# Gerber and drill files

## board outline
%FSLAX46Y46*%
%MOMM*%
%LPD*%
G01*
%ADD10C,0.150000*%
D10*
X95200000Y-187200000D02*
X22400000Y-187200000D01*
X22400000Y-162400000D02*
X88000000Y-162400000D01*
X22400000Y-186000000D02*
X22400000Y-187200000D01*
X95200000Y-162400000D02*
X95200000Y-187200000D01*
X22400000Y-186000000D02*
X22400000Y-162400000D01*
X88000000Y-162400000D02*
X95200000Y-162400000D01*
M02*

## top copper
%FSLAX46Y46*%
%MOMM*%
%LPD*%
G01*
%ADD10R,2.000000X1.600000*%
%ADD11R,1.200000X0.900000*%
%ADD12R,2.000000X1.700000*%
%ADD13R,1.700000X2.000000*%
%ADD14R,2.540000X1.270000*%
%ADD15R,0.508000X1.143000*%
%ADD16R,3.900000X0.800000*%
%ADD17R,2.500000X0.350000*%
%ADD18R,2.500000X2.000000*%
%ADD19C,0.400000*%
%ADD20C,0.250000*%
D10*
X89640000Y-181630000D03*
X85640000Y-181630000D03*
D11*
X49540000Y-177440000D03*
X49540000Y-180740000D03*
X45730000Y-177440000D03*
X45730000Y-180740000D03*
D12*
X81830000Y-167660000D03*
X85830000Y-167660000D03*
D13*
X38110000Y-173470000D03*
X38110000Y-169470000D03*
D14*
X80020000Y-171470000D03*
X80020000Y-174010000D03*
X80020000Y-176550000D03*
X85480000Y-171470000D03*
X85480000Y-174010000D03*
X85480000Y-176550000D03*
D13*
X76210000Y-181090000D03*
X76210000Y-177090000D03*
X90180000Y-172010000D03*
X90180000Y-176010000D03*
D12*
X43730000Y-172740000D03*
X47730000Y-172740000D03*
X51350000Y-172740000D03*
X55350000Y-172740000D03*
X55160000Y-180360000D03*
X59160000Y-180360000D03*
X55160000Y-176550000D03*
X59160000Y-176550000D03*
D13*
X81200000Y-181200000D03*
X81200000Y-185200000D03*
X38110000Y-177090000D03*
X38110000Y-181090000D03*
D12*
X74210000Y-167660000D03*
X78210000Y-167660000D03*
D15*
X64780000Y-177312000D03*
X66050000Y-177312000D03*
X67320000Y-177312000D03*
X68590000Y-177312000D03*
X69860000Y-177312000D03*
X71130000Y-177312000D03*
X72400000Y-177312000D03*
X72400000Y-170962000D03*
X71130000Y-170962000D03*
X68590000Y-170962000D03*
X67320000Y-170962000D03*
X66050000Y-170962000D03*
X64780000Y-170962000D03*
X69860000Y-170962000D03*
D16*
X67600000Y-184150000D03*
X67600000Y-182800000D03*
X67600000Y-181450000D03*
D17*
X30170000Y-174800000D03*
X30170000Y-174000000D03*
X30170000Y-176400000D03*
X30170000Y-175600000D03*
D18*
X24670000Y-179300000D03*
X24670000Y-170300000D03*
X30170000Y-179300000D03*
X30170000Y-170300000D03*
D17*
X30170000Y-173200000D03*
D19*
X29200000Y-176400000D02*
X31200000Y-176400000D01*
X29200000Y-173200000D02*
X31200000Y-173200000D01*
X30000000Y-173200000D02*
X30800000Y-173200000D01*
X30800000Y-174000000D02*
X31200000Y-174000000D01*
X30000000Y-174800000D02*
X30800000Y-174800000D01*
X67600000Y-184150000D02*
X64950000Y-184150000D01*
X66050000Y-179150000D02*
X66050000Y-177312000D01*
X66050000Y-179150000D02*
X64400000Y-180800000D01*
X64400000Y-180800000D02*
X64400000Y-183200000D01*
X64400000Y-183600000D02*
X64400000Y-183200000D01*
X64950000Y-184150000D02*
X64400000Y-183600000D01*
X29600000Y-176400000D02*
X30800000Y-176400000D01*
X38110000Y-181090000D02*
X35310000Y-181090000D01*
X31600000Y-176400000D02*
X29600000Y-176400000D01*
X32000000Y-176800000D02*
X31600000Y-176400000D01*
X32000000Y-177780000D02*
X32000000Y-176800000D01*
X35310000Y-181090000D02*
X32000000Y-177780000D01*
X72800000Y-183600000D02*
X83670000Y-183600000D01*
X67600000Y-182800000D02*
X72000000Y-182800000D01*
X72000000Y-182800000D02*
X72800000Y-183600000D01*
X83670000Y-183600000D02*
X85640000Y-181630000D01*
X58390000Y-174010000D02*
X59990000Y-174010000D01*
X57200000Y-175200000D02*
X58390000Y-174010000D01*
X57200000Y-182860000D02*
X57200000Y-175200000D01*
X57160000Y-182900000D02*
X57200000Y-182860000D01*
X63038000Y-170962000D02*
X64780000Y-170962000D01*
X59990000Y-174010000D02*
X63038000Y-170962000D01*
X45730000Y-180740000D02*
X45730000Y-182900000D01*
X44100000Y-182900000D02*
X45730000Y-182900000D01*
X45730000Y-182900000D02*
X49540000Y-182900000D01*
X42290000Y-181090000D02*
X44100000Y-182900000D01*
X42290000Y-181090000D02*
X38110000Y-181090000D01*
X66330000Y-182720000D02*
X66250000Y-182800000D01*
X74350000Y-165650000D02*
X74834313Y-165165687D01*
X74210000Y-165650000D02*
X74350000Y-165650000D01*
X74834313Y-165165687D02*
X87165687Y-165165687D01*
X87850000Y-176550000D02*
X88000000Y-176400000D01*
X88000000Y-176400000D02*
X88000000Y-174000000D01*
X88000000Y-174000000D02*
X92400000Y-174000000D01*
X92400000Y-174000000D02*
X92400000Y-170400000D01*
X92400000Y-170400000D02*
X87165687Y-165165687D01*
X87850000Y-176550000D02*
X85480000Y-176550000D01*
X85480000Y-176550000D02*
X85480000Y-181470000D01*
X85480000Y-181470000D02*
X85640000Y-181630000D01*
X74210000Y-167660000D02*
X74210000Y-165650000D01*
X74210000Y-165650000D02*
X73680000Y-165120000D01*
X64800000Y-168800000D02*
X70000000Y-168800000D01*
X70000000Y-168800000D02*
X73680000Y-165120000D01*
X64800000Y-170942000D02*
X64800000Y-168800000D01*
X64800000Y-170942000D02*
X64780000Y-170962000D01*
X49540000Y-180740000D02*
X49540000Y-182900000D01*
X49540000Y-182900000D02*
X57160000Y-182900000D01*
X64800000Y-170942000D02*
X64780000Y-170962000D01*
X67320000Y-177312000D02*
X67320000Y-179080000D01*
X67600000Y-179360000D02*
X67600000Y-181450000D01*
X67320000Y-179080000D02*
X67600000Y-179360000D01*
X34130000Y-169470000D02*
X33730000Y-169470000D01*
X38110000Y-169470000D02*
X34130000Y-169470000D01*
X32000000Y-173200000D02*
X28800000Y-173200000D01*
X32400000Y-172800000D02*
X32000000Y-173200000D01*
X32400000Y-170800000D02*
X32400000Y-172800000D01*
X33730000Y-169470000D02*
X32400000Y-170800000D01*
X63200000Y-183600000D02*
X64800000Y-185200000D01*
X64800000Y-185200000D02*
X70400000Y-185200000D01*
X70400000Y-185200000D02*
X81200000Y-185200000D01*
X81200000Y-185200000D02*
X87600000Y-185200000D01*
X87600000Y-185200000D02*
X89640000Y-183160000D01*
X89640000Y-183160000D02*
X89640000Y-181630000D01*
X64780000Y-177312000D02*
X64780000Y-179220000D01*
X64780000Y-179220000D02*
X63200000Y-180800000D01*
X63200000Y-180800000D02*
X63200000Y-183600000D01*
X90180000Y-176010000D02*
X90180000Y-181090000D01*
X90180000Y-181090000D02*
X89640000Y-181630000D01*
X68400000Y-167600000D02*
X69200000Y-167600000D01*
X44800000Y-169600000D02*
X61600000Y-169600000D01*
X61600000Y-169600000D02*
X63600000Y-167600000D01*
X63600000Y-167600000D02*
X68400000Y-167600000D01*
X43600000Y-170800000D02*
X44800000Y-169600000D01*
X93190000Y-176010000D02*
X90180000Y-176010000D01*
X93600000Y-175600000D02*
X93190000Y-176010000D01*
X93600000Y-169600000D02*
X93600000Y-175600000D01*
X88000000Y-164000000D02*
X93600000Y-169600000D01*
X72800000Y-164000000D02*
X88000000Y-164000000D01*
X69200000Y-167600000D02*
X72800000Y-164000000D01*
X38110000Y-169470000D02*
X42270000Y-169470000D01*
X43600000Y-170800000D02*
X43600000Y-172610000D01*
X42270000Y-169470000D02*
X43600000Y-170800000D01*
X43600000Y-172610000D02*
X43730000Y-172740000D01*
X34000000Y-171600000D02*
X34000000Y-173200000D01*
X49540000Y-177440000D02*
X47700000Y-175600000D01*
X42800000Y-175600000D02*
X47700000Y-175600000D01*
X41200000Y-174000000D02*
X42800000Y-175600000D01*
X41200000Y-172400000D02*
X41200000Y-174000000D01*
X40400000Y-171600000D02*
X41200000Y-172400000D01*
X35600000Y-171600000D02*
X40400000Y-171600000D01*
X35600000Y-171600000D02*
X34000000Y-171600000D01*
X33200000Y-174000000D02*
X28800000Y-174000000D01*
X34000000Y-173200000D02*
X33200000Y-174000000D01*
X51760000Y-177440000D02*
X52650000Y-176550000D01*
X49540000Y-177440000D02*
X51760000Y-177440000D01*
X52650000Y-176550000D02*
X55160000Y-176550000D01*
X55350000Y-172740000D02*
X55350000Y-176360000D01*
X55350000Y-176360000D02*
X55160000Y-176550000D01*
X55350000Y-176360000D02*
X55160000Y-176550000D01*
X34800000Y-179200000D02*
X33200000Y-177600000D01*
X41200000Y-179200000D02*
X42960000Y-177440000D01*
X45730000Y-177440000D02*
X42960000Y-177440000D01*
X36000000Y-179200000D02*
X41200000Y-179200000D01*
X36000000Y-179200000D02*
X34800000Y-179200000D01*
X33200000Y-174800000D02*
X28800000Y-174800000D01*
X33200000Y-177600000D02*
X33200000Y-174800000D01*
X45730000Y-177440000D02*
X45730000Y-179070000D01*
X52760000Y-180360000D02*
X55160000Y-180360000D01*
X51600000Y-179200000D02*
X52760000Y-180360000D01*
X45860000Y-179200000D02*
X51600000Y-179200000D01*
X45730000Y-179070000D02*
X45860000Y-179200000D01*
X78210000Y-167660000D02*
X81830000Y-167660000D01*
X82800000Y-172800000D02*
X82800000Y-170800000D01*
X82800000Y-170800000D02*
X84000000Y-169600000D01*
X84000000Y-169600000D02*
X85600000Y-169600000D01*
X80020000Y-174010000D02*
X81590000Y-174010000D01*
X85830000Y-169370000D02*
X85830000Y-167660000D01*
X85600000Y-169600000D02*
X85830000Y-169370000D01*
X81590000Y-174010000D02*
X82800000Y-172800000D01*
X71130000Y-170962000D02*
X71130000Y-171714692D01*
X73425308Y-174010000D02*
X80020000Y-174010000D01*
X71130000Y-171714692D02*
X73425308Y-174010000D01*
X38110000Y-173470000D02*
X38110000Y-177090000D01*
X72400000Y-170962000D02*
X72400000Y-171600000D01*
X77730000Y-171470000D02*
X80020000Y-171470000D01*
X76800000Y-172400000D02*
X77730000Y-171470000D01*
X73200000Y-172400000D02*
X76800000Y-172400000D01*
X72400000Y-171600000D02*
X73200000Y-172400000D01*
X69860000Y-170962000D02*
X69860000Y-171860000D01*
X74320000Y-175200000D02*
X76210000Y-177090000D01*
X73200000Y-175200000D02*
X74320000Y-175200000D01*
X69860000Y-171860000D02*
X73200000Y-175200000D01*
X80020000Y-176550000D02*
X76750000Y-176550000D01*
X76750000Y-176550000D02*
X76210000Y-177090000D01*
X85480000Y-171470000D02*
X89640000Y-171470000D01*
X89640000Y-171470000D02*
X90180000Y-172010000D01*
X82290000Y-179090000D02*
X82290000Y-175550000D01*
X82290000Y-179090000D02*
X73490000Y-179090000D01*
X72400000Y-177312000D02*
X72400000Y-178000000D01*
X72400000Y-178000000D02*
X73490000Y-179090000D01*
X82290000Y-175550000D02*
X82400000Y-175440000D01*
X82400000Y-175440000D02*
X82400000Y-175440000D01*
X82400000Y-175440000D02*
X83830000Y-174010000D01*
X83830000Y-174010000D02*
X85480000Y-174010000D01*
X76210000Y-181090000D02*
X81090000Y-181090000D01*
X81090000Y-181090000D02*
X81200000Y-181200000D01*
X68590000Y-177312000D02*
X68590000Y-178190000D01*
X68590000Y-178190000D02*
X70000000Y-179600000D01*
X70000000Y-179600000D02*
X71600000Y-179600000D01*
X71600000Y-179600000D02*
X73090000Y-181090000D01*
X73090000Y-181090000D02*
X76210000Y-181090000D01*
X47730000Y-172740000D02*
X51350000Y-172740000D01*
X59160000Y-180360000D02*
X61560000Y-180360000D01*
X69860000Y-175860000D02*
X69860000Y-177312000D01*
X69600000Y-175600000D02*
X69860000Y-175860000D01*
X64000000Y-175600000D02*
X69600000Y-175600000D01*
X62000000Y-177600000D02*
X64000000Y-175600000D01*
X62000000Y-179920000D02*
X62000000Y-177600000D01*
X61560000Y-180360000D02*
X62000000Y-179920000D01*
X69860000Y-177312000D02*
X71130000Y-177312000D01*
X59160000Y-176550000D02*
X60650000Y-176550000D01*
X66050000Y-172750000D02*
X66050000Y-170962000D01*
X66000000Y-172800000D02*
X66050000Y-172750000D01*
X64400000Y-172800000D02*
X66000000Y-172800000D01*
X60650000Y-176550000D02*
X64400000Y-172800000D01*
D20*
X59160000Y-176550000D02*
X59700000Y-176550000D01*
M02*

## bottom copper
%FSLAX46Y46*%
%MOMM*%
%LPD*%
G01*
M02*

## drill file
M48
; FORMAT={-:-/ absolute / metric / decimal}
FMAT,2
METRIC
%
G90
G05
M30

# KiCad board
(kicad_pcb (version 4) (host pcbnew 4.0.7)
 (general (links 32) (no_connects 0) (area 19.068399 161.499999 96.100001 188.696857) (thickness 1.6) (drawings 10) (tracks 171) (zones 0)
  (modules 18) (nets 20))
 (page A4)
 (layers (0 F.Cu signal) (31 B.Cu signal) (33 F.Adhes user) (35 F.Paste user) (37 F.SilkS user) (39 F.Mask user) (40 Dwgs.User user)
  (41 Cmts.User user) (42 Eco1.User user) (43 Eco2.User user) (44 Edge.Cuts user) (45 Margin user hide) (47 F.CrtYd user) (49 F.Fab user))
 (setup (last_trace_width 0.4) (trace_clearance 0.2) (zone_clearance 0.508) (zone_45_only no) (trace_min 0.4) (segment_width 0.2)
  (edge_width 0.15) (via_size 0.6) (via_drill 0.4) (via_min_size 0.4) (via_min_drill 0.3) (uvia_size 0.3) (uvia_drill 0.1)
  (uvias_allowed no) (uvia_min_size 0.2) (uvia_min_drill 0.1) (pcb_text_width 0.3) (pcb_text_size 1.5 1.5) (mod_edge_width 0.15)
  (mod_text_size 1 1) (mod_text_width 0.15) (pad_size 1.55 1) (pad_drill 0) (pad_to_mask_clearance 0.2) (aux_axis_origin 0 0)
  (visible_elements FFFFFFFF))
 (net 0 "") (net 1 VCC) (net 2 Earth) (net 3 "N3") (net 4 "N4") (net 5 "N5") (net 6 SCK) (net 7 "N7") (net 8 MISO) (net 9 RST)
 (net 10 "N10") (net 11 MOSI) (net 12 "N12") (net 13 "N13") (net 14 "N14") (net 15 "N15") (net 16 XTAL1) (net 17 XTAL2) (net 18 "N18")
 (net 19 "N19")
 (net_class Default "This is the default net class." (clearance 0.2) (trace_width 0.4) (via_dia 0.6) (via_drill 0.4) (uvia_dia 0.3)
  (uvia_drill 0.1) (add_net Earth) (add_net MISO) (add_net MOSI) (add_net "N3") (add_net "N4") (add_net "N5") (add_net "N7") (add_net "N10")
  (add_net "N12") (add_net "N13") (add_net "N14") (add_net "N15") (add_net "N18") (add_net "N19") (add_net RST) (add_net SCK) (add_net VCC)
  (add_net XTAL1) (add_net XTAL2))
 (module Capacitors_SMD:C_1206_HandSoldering (layer F.Cu) (at 87.64 181.63 180)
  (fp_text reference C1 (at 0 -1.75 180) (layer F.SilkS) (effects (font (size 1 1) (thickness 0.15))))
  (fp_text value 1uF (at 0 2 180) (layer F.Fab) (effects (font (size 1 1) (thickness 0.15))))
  (pad 1 smd rect (at -2 0 180) (size 2 1.6) (layers F.Cu F.Paste F.Mask) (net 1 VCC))
  (pad 2 smd rect (at 2 0 180) (size 2 1.6) (layers F.Cu F.Paste F.Mask) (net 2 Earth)))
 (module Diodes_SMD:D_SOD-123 (layer F.Cu) (at 49.54 179.09 270)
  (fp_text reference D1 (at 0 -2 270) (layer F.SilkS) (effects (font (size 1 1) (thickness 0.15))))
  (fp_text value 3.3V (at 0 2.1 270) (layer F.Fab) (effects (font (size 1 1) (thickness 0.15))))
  (pad 1 smd rect (at -1.65 0 270) (size 0.9 1.2) (layers F.Cu F.Paste F.Mask) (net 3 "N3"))
  (pad 2 smd rect (at 1.65 0 270) (size 0.9 1.2) (layers F.Cu F.Paste F.Mask) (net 2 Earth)))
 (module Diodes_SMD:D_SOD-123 (layer F.Cu) (at 45.73 179.09 270)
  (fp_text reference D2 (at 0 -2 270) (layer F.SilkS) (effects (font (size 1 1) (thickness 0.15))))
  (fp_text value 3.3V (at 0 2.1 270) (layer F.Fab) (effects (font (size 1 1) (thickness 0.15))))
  (pad 1 smd rect (at -1.65 0 270) (size 0.9 1.2) (layers F.Cu F.Paste F.Mask) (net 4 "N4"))
  (pad 2 smd rect (at 1.65 0 270) (size 0.9 1.2) (layers F.Cu F.Paste F.Mask) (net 2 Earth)))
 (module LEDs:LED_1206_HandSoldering (layer F.Cu) (at 83.83 167.66)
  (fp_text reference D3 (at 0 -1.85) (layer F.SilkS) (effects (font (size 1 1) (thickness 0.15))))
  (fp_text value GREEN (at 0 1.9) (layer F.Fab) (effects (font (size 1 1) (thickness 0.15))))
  (pad 1 smd rect (at -2 0) (size 2 1.7) (layers F.Cu F.Paste F.Mask) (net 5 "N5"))
  (pad 2 smd rect (at 2 0) (size 2 1.7) (layers F.Cu F.Paste F.Mask) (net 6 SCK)))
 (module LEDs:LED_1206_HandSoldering (layer F.Cu) (at 38.11 171.47 90)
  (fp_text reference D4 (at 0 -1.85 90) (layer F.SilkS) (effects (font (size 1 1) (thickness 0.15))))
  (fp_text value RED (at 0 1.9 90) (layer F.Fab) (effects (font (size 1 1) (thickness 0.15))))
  (pad 1 smd rect (at -2 0 90) (size 2 1.7) (layers F.Cu F.Paste F.Mask) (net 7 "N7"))
  (pad 2 smd rect (at 2 0 90) (size 2 1.7) (layers F.Cu F.Paste F.Mask) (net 1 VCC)))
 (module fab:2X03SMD (layer F.Cu) (at 82.56 174.01)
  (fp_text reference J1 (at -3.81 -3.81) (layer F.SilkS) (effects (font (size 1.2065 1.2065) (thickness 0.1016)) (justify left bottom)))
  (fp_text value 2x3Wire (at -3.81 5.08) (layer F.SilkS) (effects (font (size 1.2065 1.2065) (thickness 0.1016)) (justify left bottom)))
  (pad 1 smd rect (at -2.54 -2.54) (size 2.54 1.27) (layers F.Cu F.Paste F.Mask) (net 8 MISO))
  (pad 3 smd rect (at -2.54 0) (size 2.54 1.27) (layers F.Cu F.Paste F.Mask) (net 6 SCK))
  (pad 5 smd rect (at -2.54 2.54) (size 2.54 1.27) (layers F.Cu F.Paste F.Mask) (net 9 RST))
  (pad 2 smd rect (at 2.92 -2.54) (size 2.54 1.27) (layers F.Cu F.Paste F.Mask) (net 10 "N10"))
  (pad 4 smd rect (at 2.92 0) (size 2.54 1.27) (layers F.Cu F.Paste F.Mask) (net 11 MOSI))
  (pad 6 smd rect (at 2.92 2.54) (size 2.54 1.27) (layers F.Cu F.Paste F.Mask) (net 2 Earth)))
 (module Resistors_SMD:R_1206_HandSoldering (layer F.Cu) (at 76.21 179.09 90)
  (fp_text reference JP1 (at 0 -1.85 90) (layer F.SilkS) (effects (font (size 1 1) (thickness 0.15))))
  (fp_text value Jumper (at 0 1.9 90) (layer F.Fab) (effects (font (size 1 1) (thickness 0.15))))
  (pad 1 smd rect (at -2 0 90) (size 2 1.7) (layers F.Cu F.Paste F.Mask) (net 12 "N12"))
  (pad 2 smd rect (at 2 0 90) (size 2 1.7) (layers F.Cu F.Paste F.Mask) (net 9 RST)))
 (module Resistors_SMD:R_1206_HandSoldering (layer F.Cu) (at 90.18 174.01 270)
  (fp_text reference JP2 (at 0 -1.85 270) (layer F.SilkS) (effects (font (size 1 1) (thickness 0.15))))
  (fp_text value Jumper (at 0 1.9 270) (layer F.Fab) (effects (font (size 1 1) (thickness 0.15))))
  (pad 1 smd rect (at -2 0 270) (size 2 1.7) (layers F.Cu F.Paste F.Mask) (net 10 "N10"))
  (pad 2 smd rect (at 2 0 270) (size 2 1.7) (layers F.Cu F.Paste F.Mask) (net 1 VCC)))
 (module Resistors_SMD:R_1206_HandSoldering (layer F.Cu) (at 45.73 172.74)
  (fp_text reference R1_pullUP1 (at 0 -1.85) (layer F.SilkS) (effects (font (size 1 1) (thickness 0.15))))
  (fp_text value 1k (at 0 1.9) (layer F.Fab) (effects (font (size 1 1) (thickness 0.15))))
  (pad 1 smd rect (at -2 0) (size 2 1.7) (layers F.Cu F.Paste F.Mask) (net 1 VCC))
  (pad 2 smd rect (at 2 0) (size 2 1.7) (layers F.Cu F.Paste F.Mask) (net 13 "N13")))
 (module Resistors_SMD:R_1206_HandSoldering (layer F.Cu) (at 53.35 172.74)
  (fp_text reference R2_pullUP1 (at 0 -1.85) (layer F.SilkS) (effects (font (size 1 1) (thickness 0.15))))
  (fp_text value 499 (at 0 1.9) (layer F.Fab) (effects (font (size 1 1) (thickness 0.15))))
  (pad 1 smd rect (at -2 0) (size 2 1.7) (layers F.Cu F.Paste F.Mask) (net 13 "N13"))
  (pad 2 smd rect (at 2 0) (size 2 1.7) (layers F.Cu F.Paste F.Mask) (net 3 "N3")))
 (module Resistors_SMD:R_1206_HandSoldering (layer F.Cu) (at 57.16 180.36)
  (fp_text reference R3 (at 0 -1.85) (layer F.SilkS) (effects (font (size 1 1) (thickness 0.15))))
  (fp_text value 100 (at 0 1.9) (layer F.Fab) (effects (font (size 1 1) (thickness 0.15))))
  (pad 1 smd rect (at -2 0) (size 2 1.7) (layers F.Cu F.Paste F.Mask) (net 4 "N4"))
  (pad 2 smd rect (at 2 0) (size 2 1.7) (layers F.Cu F.Paste F.Mask) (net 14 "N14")))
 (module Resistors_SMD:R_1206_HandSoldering (layer F.Cu) (at 57.16 176.55)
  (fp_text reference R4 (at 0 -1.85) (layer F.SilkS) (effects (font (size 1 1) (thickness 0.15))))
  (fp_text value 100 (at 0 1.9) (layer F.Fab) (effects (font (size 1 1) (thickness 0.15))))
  (pad 1 smd rect (at -2 0) (size 2 1.7) (layers F.Cu F.Paste F.Mask) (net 3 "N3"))
  (pad 2 smd rect (at 2 0) (size 2 1.7) (layers F.Cu F.Paste F.Mask) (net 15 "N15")))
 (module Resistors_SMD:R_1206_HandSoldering (layer F.Cu) (at 81.2 183.2 270)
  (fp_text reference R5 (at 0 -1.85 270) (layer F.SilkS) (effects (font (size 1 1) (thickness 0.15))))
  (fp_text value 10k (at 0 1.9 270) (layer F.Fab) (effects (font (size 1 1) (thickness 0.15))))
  (pad 1 smd rect (at -2 0 270) (size 2 1.7) (layers F.Cu F.Paste F.Mask) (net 12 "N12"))
  (pad 2 smd rect (at 2 0 270) (size 2 1.7) (layers F.Cu F.Paste F.Mask) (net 1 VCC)))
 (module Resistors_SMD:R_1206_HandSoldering (layer F.Cu) (at 38.11 179.09 270)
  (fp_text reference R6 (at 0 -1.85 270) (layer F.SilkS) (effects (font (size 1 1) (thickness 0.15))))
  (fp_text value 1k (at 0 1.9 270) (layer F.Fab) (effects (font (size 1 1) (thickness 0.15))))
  (pad 1 smd rect (at -2 0 270) (size 2 1.7) (layers F.Cu F.Paste F.Mask) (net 7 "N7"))
  (pad 2 smd rect (at 2 0 270) (size 2 1.7) (layers F.Cu F.Paste F.Mask) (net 2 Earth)))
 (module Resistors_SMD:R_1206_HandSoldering (layer F.Cu) (at 76.21 167.66)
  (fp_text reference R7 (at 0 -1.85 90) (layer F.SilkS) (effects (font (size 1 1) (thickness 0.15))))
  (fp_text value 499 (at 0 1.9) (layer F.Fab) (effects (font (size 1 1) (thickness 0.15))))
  (pad 1 smd rect (at -2 0) (size 2 1.7) (layers F.Cu F.Paste F.Mask) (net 2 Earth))
  (pad 2 smd rect (at 2 0) (size 2 1.7) (layers F.Cu F.Paste F.Mask) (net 5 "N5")))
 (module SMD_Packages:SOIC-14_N (layer F.Cu) (at 68.59 174.01)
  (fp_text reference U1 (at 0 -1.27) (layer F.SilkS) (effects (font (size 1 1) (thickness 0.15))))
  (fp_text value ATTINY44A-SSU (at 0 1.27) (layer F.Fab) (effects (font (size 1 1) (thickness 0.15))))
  (pad 1 smd rect (at -3.81 3.302) (size 0.508 1.143) (layers F.Cu F.Paste F.Mask) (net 1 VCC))
  (pad 2 smd rect (at -2.54 3.302) (size 0.508 1.143) (layers F.Cu F.Paste F.Mask) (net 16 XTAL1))
  (pad 3 smd rect (at -1.27 3.302) (size 0.508 1.143) (layers F.Cu F.Paste F.Mask) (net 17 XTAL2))
  (pad 4 smd rect (at 0 3.302) (size 0.508 1.143) (layers F.Cu F.Paste F.Mask) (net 12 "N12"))
  (pad 5 smd rect (at 1.27 3.302) (size 0.508 1.143) (layers F.Cu F.Paste F.Mask) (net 14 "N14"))
  (pad 6 smd rect (at 2.54 3.302) (size 0.508 1.143) (layers F.Cu F.Paste F.Mask) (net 14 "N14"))
  (pad 7 smd rect (at 3.81 3.302) (size 0.508 1.143) (layers F.Cu F.Paste F.Mask) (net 11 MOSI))
  (pad 8 smd rect (at 3.81 -3.048) (size 0.508 1.143) (layers F.Cu F.Paste F.Mask) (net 8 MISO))
  (pad 9 smd rect (at 2.54 -3.048) (size 0.508 1.143) (layers F.Cu F.Paste F.Mask) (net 6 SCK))
  (pad 11 smd rect (at 0 -3.048) (size 0.508 1.143) (layers F.Cu F.Paste F.Mask) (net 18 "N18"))
  (pad 12 smd rect (at -1.27 -3.048) (size 0.508 1.143) (layers F.Cu F.Paste F.Mask) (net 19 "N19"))
  (pad 13 smd rect (at -2.54 -3.048) (size 0.508 1.143) (layers F.Cu F.Paste F.Mask) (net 15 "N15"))
  (pad 14 smd rect (at -3.81 -3.048) (size 0.508 1.143) (layers F.Cu F.Paste F.Mask) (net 2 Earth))
  (pad 10 smd rect (at 1.27 -3.048) (size 0.508 1.143) (layers F.Cu F.Paste F.Mask) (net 9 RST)))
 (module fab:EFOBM (layer F.Cu) (at 67.6 182.8 90)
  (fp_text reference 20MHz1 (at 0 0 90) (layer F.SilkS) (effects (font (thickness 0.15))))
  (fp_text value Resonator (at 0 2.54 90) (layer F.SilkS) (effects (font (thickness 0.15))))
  (pad 1 smd rect (at -1.35 0 180) (size 3.9 0.8) (layers F.Cu F.Paste F.Mask) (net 16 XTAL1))
  (pad 2 smd rect (at 0 0) (size 3.9 0.8) (layers F.Cu F.Paste F.Mask) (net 2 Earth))
  (pad 3 smd rect (at 1.35 0) (size 3.9 0.8) (layers F.Cu F.Paste F.Mask) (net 17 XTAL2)))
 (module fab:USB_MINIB (layer F.Cu) (at 26.4 174.8)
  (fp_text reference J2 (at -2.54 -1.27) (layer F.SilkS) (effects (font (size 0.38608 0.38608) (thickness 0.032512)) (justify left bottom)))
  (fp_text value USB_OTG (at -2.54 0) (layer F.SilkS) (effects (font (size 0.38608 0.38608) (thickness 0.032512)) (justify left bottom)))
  (pad D+ smd rect (at 3.77 0) (size 2.5 0.35) (layers F.Cu F.Paste F.Mask))
  (pad D- smd rect (at 3.77 -0.8) (size 2.5 0.35) (layers F.Cu F.Paste F.Mask))
  (pad GND smd rect (at 3.77 1.6) (size 2.5 0.35) (layers F.Cu F.Paste F.Mask))
  (pad ID smd rect (at 3.77 0.8) (size 2.5 0.35) (layers F.Cu F.Paste F.Mask))
  (pad SHIE smd rect (at -1.73 4.5) (size 2.5 2) (layers F.Cu F.Paste F.Mask))
  (pad SHIE smd rect (at -1.73 -4.5) (size 2.5 2) (layers F.Cu F.Paste F.Mask))
  (pad SHIE smd rect (at 3.77 4.5) (size 2.5 2) (layers F.Cu F.Paste F.Mask))
  (pad SHIE smd rect (at 3.77 -4.5) (size 2.5 2) (layers F.Cu F.Paste F.Mask))
  (pad VBUS smd rect (at 3.77 -1.6) (size 2.5 0.35) (layers F.Cu F.Paste F.Mask)))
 (gr_line (start 95.2 187.2) (end 22.4 187.2) (angle 90) (layer Edge.Cuts) (width 0.15))
 (gr_line (start 22.4 162.4) (end 88 162.4) (angle 90) (layer Edge.Cuts) (width 0.15))
 (gr_line (start 22.4 186) (end 22.4 187.2) (angle 90) (layer Edge.Cuts) (width 0.15))
 (gr_line (start 95.2 162.4) (end 95.2 187.2) (angle 90) (layer Edge.Cuts) (width 0.15))
 (gr_line (start 22.4 186) (end 22.4 162.4) (angle 90) (layer Edge.Cuts) (width 0.15))
 (gr_line (start 88 162.4) (end 95.2 162.4) (angle 90) (layer Edge.Cuts) (width 0.15))
 (segment (start 29.2 176.4) (end 31.2 176.4) (width 0.4) (layer F.Cu) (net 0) (status 30))
 (segment (start 29.2 173.2) (end 31.2 173.2) (width 0.4) (layer F.Cu) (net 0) (status 30))
 (segment (start 30 173.2) (end 30.8 173.2) (width 0.4) (layer F.Cu) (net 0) (status 30))
 (segment (start 30.8 174) (end 31.2 174) (width 0.4) (layer F.Cu) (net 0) (status 30))
 (segment (start 30 174.8) (end 30.8 174.8) (width 0.4) (layer F.Cu) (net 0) (status 30))
 (segment (start 67.6 184.15) (end 64.95 184.15) (width 0.4) (layer F.Cu) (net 16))
 (segment (start 66.05 179.15) (end 66.05 177.312) (width 0.4) (layer F.Cu) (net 16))
 (segment (start 66.05 179.15) (end 64.4 180.8) (width 0.4) (layer F.Cu) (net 16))
 (segment (start 64.4 180.8) (end 64.4 183.2) (width 0.4) (layer F.Cu) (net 16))
 (segment (start 64.4 183.6) (end 64.4 183.2) (width 0.4) (layer F.Cu) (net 16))
 (segment (start 64.95 184.15) (end 64.4 183.6) (width 0.4) (layer F.Cu) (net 16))
 (segment (start 29.6 176.4) (end 30.8 176.4) (width 0.4) (layer F.Cu) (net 2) (status 30))
 (segment (start 38.11 181.09) (end 35.31 181.09) (width 0.4) (layer F.Cu) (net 2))
 (segment (start 31.6 176.4) (end 29.6 176.4) (width 0.4) (layer F.Cu) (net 2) (status 20))
 (segment (start 32 176.8) (end 31.6 176.4) (width 0.4) (layer F.Cu) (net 2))
 (segment (start 32 177.78) (end 32 176.8) (width 0.4) (layer F.Cu) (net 2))
 (segment (start 35.31 181.09) (end 32 177.78) (width 0.4) (layer F.Cu) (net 2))
 (segment (start 72.8 183.6) (end 83.67 183.6) (width 0.4) (layer F.Cu) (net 2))
 (segment (start 67.6 182.8) (end 72 182.8) (width 0.4) (layer F.Cu) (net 2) (status 10))
 (segment (start 72 182.8) (end 72.8 183.6) (width 0.4) (layer F.Cu) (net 2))
 (segment (start 83.67 183.6) (end 85.64 181.63) (width 0.4) (layer F.Cu) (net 2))
 (segment (start 58.39 174.01) (end 59.99 174.01) (width 0.4) (layer F.Cu) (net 2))
 (segment (start 57.2 175.2) (end 58.39 174.01) (width 0.4) (layer F.Cu) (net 2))
 (segment (start 57.2 182.86) (end 57.2 175.2) (width 0.4) (layer F.Cu) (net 2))
 (segment (start 57.16 182.9) (end 57.2 182.86) (width 0.4) (layer F.Cu) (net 2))
 (segment (start 63.038 170.962) (end 64.78 170.962) (width 0.4) (layer F.Cu) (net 2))
 (segment (start 59.99 174.01) (end 63.038 170.962) (width 0.4) (layer F.Cu) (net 2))
 (segment (start 45.73 180.74) (end 45.73 182.9) (width 0.4) (layer F.Cu) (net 2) (status 10))
 (segment (start 44.1 182.9) (end 45.73 182.9) (width 0.4) (layer F.Cu) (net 2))
 (segment (start 45.73 182.9) (end 49.54 182.9) (width 0.4) (layer F.Cu) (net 2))
 (segment (start 42.29 181.09) (end 44.1 182.9) (width 0.4) (layer F.Cu) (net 2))
 (segment (start 42.29 181.09) (end 38.11 181.09) (width 0.4) (layer F.Cu) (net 2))
 (segment (start 66.33 182.72) (end 66.25 182.8) (width 0.4) (layer F.Cu) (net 2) (status 30))
 (segment (start 74.35 165.65) (end 74.834313 165.165687) (width 0.4) (layer F.Cu) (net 2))
 (segment (start 74.21 165.65) (end 74.35 165.65) (width 0.4) (layer F.Cu) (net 2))
 (segment (start 74.834313 165.165687) (end 87.165687 165.165687) (width 0.4) (layer F.Cu) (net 2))
 (segment (start 87.85 176.55) (end 88 176.4) (width 0.4) (layer F.Cu) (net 2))
 (segment (start 88 176.4) (end 88 174) (width 0.4) (layer F.Cu) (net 2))
 (segment (start 88 174) (end 92.4 174) (width 0.4) (layer F.Cu) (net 2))
 (segment (start 92.4 174) (end 92.4 170.4) (width 0.4) (layer F.Cu) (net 2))
 (segment (start 92.4 170.4) (end 87.165687 165.165687) (width 0.4) (layer F.Cu) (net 2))
 (segment (start 87.85 176.55) (end 85.48 176.55) (width 0.4) (layer F.Cu) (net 2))
 (segment (start 85.48 176.55) (end 85.48 181.47) (width 0.4) (layer F.Cu) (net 2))
 (segment (start 85.48 181.47) (end 85.64 181.63) (width 0.4) (layer F.Cu) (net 2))
 (segment (start 74.21 167.66) (end 74.21 165.65) (width 0.4) (layer F.Cu) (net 2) (status 10))
 (segment (start 74.21 165.65) (end 73.68 165.12) (width 0.4) (layer F.Cu) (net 2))
 (segment (start 64.8 168.8) (end 70 168.8) (width 0.4) (layer F.Cu) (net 2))
 (segment (start 70 168.8) (end 73.68 165.12) (width 0.4) (layer F.Cu) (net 2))
 (segment (start 64.8 170.942) (end 64.8 168.8) (width 0.4) (layer F.Cu) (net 2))
 (segment (start 64.8 170.942) (end 64.78 170.962) (width 0.4) (layer F.Cu) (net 2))
 (segment (start 49.54 180.74) (end 49.54 182.9) (width 0.4) (layer F.Cu) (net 2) (status 10))
 (segment (start 49.54 182.9) (end 57.16 182.9) (width 0.4) (layer F.Cu) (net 2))
 (segment (start 64.8 170.942) (end 64.78 170.962) (width 0.4) (layer F.Cu) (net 2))
 (segment (start 67.32 177.312) (end 67.32 179.08) (width 0.4) (layer F.Cu) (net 17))
 (segment (start 67.6 179.36) (end 67.6 181.45) (width 0.4) (layer F.Cu) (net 17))
 (segment (start 67.32 179.08) (end 67.6 179.36) (width 0.4) (layer F.Cu) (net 17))
 (segment (start 34.13 169.47) (end 33.73 169.47) (width 0.4) (layer F.Cu) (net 1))
 (segment (start 38.11 169.47) (end 34.13 169.47) (width 0.4) (layer F.Cu) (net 1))
 (segment (start 32 173.2) (end 28.8 173.2) (width 0.4) (layer F.Cu) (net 1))
 (segment (start 32.4 172.8) (end 32 173.2) (width 0.4) (layer F.Cu) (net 1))
 (segment (start 32.4 170.8) (end 32.4 172.8) (width 0.4) (layer F.Cu) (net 1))
 (segment (start 33.73 169.47) (end 32.4 170.8) (width 0.4) (layer F.Cu) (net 1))
 (segment (start 63.2 183.6) (end 64.8 185.2) (width 0.4) (layer F.Cu) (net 1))
 (segment (start 64.8 185.2) (end 70.4 185.2) (width 0.4) (layer F.Cu) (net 1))
 (segment (start 70.4 185.2) (end 81.2 185.2) (width 0.4) (layer F.Cu) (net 1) (status 20))
 (segment (start 81.2 185.2) (end 87.6 185.2) (width 0.4) (layer F.Cu) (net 1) (status 10))
 (segment (start 87.6 185.2) (end 89.64 183.16) (width 0.4) (layer F.Cu) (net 1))
 (segment (start 89.64 183.16) (end 89.64 181.63) (width 0.4) (layer F.Cu) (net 1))
 (segment (start 64.78 177.312) (end 64.78 179.22) (width 0.4) (layer F.Cu) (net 1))
 (segment (start 64.78 179.22) (end 63.2 180.8) (width 0.4) (layer F.Cu) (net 1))
 (segment (start 63.2 180.8) (end 63.2 183.6) (width 0.4) (layer F.Cu) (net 1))
 (segment (start 90.18 176.01) (end 90.18 181.09) (width 0.4) (layer F.Cu) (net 1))
 (segment (start 90.18 181.09) (end 89.64 181.63) (width 0.4) (layer F.Cu) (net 1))
 (segment (start 68.4 167.6) (end 69.2 167.6) (width 0.4) (layer F.Cu) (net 1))
 (segment (start 44.8 169.6) (end 61.6 169.6) (width 0.4) (layer F.Cu) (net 1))
 (segment (start 61.6 169.6) (end 63.6 167.6) (width 0.4) (layer F.Cu) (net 1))
 (segment (start 63.6 167.6) (end 68.4 167.6) (width 0.4) (layer F.Cu) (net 1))
 (segment (start 43.6 170.8) (end 44.8 169.6) (width 0.4) (layer F.Cu) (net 1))
 (segment (start 93.19 176.01) (end 90.18 176.01) (width 0.4) (layer F.Cu) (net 1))
 (segment (start 93.6 175.6) (end 93.19 176.01) (width 0.4) (layer F.Cu) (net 1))
 (segment (start 93.6 169.6) (end 93.6 175.6) (width 0.4) (layer F.Cu) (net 1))
 (segment (start 88 164) (end 93.6 169.6) (width 0.4) (layer F.Cu) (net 1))
 (segment (start 72.8 164) (end 88 164) (width 0.4) (layer F.Cu) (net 1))
 (segment (start 69.2 167.6) (end 72.8 164) (width 0.4) (layer F.Cu) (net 1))
 (segment (start 38.11 169.47) (end 42.27 169.47) (width 0.4) (layer F.Cu) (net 1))
 (segment (start 43.6 170.8) (end 43.6 172.61) (width 0.4) (layer F.Cu) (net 1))
 (segment (start 42.27 169.47) (end 43.6 170.8) (width 0.4) (layer F.Cu) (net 1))
 (segment (start 43.6 172.61) (end 43.73 172.74) (width 0.4) (layer F.Cu) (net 1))
 (segment (start 34 171.6) (end 34 173.2) (width 0.4) (layer F.Cu) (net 3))
 (segment (start 49.54 177.44) (end 47.7 175.6) (width 0.4) (layer F.Cu) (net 3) (status 20))
 (segment (start 42.8 175.6) (end 47.7 175.6) (width 0.4) (layer F.Cu) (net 3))
 (segment (start 41.2 174) (end 42.8 175.6) (width 0.4) (layer F.Cu) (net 3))
 (segment (start 41.2 172.4) (end 41.2 174) (width 0.4) (layer F.Cu) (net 3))
 (segment (start 40.4 171.6) (end 41.2 172.4) (width 0.4) (layer F.Cu) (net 3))
 (segment (start 35.6 171.6) (end 40.4 171.6) (width 0.4) (layer F.Cu) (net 3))
 (segment (start 35.6 171.6) (end 34 171.6) (width 0.4) (layer F.Cu) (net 3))
 (segment (start 33.2 174) (end 28.8 174) (width 0.4) (layer F.Cu) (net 3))
 (segment (start 34 173.2) (end 33.2 174) (width 0.4) (layer F.Cu) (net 3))
 (segment (start 51.76 177.44) (end 52.65 176.55) (width 0.4) (layer F.Cu) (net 3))
 (segment (start 49.54 177.44) (end 51.76 177.44) (width 0.4) (layer F.Cu) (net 3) (status 10))
 (segment (start 52.65 176.55) (end 55.16 176.55) (width 0.4) (layer F.Cu) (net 3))
 (segment (start 55.35 172.74) (end 55.35 176.36) (width 0.4) (layer F.Cu) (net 3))
 (segment (start 55.35 176.36) (end 55.16 176.55) (width 0.4) (layer F.Cu) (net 3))
 (segment (start 55.35 176.36) (end 55.16 176.55) (width 0.4) (layer F.Cu) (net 3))
 (segment (start 34.8 179.2) (end 33.2 177.6) (width 0.4) (layer F.Cu) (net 4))
 (segment (start 41.2 179.2) (end 42.96 177.44) (width 0.4) (layer F.Cu) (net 4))
 (segment (start 45.73 177.44) (end 42.96 177.44) (width 0.4) (layer F.Cu) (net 4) (status 20))
 (segment (start 36 179.2) (end 41.2 179.2) (width 0.4) (layer F.Cu) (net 4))
 (segment (start 36 179.2) (end 34.8 179.2) (width 0.4) (layer F.Cu) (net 4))
 (segment (start 33.2 174.8) (end 28.8 174.8) (width 0.4) (layer F.Cu) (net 4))
 (segment (start 33.2 177.6) (end 33.2 174.8) (width 0.4) (layer F.Cu) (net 4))
 (segment (start 45.73 177.44) (end 45.73 179.07) (width 0.4) (layer F.Cu) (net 4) (status 10))
 (segment (start 52.76 180.36) (end 55.16 180.36) (width 0.4) (layer F.Cu) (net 4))
 (segment (start 51.6 179.2) (end 52.76 180.36) (width 0.4) (layer F.Cu) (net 4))
 (segment (start 45.86 179.2) (end 51.6 179.2) (width 0.4) (layer F.Cu) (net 4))
 (segment (start 45.73 179.07) (end 45.86 179.2) (width 0.4) (layer F.Cu) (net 4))
 (segment (start 78.21 167.66) (end 81.83 167.66) (width 0.4) (layer F.Cu) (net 5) (status 20))
 (segment (start 82.8 172.8) (end 82.8 170.8) (width 0.4) (layer F.Cu) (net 6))
 (segment (start 82.8 170.8) (end 84 169.6) (width 0.4) (layer F.Cu) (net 6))
 (segment (start 84 169.6) (end 85.6 169.6) (width 0.4) (layer F.Cu) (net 6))
 (segment (start 80.02 174.01) (end 81.59 174.01) (width 0.4) (layer F.Cu) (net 6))
 (segment (start 85.83 169.37) (end 85.83 167.66) (width 0.4) (layer F.Cu) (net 6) (status 20))
 (segment (start 85.6 169.6) (end 85.83 169.37) (width 0.4) (layer F.Cu) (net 6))
 (segment (start 81.59 174.01) (end 82.8 172.8) (width 0.4) (layer F.Cu) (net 6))
 (segment (start 71.13 170.962) (end 71.13 171.714692) (width 0.4) (layer F.Cu) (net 6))
 (segment (start 73.425308 174.01) (end 80.02 174.01) (width 0.4) (layer F.Cu) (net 6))
 (segment (start 71.13 171.714692) (end 73.425308 174.01) (width 0.4) (layer F.Cu) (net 6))
 (segment (start 38.11 173.47) (end 38.11 177.09) (width 0.4) (layer F.Cu) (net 7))
 (segment (start 72.4 170.962) (end 72.4 171.6) (width 0.4) (layer F.Cu) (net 8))
 (segment (start 77.73 171.47) (end 80.02 171.47) (width 0.4) (layer F.Cu) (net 8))
 (segment (start 76.8 172.4) (end 77.73 171.47) (width 0.4) (layer F.Cu) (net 8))
 (segment (start 73.2 172.4) (end 76.8 172.4) (width 0.4) (layer F.Cu) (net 8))
 (segment (start 72.4 171.6) (end 73.2 172.4) (width 0.4) (layer F.Cu) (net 8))
 (segment (start 69.86 170.962) (end 69.86 171.86) (width 0.4) (layer F.Cu) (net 9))
 (segment (start 74.32 175.2) (end 76.21 177.09) (width 0.4) (layer F.Cu) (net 9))
 (segment (start 73.2 175.2) (end 74.32 175.2) (width 0.4) (layer F.Cu) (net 9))
 (segment (start 69.86 171.86) (end 73.2 175.2) (width 0.4) (layer F.Cu) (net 9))
 (segment (start 80.02 176.55) (end 76.75 176.55) (width 0.4) (layer F.Cu) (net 9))
 (segment (start 76.75 176.55) (end 76.21 177.09) (width 0.4) (layer F.Cu) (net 9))
 (segment (start 85.48 171.47) (end 89.64 171.47) (width 0.4) (layer F.Cu) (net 10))
 (segment (start 89.64 171.47) (end 90.18 172.01) (width 0.4) (layer F.Cu) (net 10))
 (segment (start 82.29 179.09) (end 82.29 175.55) (width 0.4) (layer F.Cu) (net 11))
 (segment (start 82.29 179.09) (end 73.49 179.09) (width 0.4) (layer F.Cu) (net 11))
 (segment (start 72.4 177.312) (end 72.4 178) (width 0.4) (layer F.Cu) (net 11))
 (segment (start 72.4 178) (end 73.49 179.09) (width 0.4) (layer F.Cu) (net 11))
 (segment (start 82.29 175.55) (end 82.4 175.44) (width 0.4) (layer F.Cu) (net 11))
 (segment (start 82.4 175.44) (end 82.4 175.44) (width 0.4) (layer F.Cu) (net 11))
 (segment (start 82.4 175.44) (end 83.83 174.01) (width 0.4) (layer F.Cu) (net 11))
 (segment (start 83.83 174.01) (end 85.48 174.01) (width 0.4) (layer F.Cu) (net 11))
 (segment (start 76.21 181.09) (end 81.09 181.09) (width 0.4) (layer F.Cu) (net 12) (status 20))
 (segment (start 81.09 181.09) (end 81.2 181.2) (width 0.4) (layer F.Cu) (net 12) (status 30))
 (segment (start 68.59 177.312) (end 68.59 178.19) (width 0.4) (layer F.Cu) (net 12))
 (segment (start 68.59 178.19) (end 70 179.6) (width 0.4) (layer F.Cu) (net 12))
 (segment (start 70 179.6) (end 71.6 179.6) (width 0.4) (layer F.Cu) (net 12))
 (segment (start 71.6 179.6) (end 73.09 181.09) (width 0.4) (layer F.Cu) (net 12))
 (segment (start 73.09 181.09) (end 76.21 181.09) (width 0.4) (layer F.Cu) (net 12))
 (segment (start 47.73 172.74) (end 51.35 172.74) (width 0.4) (layer F.Cu) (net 13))
 (segment (start 59.16 180.36) (end 61.56 180.36) (width 0.4) (layer F.Cu) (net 14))
 (segment (start 69.86 175.86) (end 69.86 177.312) (width 0.4) (layer F.Cu) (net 14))
 (segment (start 69.6 175.6) (end 69.86 175.86) (width 0.4) (layer F.Cu) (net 14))
 (segment (start 64 175.6) (end 69.6 175.6) (width 0.4) (layer F.Cu) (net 14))
 (segment (start 62 177.6) (end 64 175.6) (width 0.4) (layer F.Cu) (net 14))
 (segment (start 62 179.92) (end 62 177.6) (width 0.4) (layer F.Cu) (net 14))
 (segment (start 61.56 180.36) (end 62 179.92) (width 0.4) (layer F.Cu) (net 14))
 (segment (start 69.86 177.312) (end 71.13 177.312) (width 0.4) (layer F.Cu) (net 14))
 (segment (start 59.16 176.55) (end 60.65 176.55) (width 0.4) (layer F.Cu) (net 15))
 (segment (start 66.05 172.75) (end 66.05 170.962) (width 0.4) (layer F.Cu) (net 15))
 (segment (start 66 172.8) (end 66.05 172.75) (width 0.4) (layer F.Cu) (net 15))
 (segment (start 64.4 172.8) (end 66 172.8) (width 0.4) (layer F.Cu) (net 15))
 (segment (start 60.65 176.55) (end 64.4 172.8) (width 0.4) (layer F.Cu) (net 15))
 (segment (start 59.16 176.55) (end 59.7 176.55) (width 0.25) (layer F.Cu) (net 15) (status 30)))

